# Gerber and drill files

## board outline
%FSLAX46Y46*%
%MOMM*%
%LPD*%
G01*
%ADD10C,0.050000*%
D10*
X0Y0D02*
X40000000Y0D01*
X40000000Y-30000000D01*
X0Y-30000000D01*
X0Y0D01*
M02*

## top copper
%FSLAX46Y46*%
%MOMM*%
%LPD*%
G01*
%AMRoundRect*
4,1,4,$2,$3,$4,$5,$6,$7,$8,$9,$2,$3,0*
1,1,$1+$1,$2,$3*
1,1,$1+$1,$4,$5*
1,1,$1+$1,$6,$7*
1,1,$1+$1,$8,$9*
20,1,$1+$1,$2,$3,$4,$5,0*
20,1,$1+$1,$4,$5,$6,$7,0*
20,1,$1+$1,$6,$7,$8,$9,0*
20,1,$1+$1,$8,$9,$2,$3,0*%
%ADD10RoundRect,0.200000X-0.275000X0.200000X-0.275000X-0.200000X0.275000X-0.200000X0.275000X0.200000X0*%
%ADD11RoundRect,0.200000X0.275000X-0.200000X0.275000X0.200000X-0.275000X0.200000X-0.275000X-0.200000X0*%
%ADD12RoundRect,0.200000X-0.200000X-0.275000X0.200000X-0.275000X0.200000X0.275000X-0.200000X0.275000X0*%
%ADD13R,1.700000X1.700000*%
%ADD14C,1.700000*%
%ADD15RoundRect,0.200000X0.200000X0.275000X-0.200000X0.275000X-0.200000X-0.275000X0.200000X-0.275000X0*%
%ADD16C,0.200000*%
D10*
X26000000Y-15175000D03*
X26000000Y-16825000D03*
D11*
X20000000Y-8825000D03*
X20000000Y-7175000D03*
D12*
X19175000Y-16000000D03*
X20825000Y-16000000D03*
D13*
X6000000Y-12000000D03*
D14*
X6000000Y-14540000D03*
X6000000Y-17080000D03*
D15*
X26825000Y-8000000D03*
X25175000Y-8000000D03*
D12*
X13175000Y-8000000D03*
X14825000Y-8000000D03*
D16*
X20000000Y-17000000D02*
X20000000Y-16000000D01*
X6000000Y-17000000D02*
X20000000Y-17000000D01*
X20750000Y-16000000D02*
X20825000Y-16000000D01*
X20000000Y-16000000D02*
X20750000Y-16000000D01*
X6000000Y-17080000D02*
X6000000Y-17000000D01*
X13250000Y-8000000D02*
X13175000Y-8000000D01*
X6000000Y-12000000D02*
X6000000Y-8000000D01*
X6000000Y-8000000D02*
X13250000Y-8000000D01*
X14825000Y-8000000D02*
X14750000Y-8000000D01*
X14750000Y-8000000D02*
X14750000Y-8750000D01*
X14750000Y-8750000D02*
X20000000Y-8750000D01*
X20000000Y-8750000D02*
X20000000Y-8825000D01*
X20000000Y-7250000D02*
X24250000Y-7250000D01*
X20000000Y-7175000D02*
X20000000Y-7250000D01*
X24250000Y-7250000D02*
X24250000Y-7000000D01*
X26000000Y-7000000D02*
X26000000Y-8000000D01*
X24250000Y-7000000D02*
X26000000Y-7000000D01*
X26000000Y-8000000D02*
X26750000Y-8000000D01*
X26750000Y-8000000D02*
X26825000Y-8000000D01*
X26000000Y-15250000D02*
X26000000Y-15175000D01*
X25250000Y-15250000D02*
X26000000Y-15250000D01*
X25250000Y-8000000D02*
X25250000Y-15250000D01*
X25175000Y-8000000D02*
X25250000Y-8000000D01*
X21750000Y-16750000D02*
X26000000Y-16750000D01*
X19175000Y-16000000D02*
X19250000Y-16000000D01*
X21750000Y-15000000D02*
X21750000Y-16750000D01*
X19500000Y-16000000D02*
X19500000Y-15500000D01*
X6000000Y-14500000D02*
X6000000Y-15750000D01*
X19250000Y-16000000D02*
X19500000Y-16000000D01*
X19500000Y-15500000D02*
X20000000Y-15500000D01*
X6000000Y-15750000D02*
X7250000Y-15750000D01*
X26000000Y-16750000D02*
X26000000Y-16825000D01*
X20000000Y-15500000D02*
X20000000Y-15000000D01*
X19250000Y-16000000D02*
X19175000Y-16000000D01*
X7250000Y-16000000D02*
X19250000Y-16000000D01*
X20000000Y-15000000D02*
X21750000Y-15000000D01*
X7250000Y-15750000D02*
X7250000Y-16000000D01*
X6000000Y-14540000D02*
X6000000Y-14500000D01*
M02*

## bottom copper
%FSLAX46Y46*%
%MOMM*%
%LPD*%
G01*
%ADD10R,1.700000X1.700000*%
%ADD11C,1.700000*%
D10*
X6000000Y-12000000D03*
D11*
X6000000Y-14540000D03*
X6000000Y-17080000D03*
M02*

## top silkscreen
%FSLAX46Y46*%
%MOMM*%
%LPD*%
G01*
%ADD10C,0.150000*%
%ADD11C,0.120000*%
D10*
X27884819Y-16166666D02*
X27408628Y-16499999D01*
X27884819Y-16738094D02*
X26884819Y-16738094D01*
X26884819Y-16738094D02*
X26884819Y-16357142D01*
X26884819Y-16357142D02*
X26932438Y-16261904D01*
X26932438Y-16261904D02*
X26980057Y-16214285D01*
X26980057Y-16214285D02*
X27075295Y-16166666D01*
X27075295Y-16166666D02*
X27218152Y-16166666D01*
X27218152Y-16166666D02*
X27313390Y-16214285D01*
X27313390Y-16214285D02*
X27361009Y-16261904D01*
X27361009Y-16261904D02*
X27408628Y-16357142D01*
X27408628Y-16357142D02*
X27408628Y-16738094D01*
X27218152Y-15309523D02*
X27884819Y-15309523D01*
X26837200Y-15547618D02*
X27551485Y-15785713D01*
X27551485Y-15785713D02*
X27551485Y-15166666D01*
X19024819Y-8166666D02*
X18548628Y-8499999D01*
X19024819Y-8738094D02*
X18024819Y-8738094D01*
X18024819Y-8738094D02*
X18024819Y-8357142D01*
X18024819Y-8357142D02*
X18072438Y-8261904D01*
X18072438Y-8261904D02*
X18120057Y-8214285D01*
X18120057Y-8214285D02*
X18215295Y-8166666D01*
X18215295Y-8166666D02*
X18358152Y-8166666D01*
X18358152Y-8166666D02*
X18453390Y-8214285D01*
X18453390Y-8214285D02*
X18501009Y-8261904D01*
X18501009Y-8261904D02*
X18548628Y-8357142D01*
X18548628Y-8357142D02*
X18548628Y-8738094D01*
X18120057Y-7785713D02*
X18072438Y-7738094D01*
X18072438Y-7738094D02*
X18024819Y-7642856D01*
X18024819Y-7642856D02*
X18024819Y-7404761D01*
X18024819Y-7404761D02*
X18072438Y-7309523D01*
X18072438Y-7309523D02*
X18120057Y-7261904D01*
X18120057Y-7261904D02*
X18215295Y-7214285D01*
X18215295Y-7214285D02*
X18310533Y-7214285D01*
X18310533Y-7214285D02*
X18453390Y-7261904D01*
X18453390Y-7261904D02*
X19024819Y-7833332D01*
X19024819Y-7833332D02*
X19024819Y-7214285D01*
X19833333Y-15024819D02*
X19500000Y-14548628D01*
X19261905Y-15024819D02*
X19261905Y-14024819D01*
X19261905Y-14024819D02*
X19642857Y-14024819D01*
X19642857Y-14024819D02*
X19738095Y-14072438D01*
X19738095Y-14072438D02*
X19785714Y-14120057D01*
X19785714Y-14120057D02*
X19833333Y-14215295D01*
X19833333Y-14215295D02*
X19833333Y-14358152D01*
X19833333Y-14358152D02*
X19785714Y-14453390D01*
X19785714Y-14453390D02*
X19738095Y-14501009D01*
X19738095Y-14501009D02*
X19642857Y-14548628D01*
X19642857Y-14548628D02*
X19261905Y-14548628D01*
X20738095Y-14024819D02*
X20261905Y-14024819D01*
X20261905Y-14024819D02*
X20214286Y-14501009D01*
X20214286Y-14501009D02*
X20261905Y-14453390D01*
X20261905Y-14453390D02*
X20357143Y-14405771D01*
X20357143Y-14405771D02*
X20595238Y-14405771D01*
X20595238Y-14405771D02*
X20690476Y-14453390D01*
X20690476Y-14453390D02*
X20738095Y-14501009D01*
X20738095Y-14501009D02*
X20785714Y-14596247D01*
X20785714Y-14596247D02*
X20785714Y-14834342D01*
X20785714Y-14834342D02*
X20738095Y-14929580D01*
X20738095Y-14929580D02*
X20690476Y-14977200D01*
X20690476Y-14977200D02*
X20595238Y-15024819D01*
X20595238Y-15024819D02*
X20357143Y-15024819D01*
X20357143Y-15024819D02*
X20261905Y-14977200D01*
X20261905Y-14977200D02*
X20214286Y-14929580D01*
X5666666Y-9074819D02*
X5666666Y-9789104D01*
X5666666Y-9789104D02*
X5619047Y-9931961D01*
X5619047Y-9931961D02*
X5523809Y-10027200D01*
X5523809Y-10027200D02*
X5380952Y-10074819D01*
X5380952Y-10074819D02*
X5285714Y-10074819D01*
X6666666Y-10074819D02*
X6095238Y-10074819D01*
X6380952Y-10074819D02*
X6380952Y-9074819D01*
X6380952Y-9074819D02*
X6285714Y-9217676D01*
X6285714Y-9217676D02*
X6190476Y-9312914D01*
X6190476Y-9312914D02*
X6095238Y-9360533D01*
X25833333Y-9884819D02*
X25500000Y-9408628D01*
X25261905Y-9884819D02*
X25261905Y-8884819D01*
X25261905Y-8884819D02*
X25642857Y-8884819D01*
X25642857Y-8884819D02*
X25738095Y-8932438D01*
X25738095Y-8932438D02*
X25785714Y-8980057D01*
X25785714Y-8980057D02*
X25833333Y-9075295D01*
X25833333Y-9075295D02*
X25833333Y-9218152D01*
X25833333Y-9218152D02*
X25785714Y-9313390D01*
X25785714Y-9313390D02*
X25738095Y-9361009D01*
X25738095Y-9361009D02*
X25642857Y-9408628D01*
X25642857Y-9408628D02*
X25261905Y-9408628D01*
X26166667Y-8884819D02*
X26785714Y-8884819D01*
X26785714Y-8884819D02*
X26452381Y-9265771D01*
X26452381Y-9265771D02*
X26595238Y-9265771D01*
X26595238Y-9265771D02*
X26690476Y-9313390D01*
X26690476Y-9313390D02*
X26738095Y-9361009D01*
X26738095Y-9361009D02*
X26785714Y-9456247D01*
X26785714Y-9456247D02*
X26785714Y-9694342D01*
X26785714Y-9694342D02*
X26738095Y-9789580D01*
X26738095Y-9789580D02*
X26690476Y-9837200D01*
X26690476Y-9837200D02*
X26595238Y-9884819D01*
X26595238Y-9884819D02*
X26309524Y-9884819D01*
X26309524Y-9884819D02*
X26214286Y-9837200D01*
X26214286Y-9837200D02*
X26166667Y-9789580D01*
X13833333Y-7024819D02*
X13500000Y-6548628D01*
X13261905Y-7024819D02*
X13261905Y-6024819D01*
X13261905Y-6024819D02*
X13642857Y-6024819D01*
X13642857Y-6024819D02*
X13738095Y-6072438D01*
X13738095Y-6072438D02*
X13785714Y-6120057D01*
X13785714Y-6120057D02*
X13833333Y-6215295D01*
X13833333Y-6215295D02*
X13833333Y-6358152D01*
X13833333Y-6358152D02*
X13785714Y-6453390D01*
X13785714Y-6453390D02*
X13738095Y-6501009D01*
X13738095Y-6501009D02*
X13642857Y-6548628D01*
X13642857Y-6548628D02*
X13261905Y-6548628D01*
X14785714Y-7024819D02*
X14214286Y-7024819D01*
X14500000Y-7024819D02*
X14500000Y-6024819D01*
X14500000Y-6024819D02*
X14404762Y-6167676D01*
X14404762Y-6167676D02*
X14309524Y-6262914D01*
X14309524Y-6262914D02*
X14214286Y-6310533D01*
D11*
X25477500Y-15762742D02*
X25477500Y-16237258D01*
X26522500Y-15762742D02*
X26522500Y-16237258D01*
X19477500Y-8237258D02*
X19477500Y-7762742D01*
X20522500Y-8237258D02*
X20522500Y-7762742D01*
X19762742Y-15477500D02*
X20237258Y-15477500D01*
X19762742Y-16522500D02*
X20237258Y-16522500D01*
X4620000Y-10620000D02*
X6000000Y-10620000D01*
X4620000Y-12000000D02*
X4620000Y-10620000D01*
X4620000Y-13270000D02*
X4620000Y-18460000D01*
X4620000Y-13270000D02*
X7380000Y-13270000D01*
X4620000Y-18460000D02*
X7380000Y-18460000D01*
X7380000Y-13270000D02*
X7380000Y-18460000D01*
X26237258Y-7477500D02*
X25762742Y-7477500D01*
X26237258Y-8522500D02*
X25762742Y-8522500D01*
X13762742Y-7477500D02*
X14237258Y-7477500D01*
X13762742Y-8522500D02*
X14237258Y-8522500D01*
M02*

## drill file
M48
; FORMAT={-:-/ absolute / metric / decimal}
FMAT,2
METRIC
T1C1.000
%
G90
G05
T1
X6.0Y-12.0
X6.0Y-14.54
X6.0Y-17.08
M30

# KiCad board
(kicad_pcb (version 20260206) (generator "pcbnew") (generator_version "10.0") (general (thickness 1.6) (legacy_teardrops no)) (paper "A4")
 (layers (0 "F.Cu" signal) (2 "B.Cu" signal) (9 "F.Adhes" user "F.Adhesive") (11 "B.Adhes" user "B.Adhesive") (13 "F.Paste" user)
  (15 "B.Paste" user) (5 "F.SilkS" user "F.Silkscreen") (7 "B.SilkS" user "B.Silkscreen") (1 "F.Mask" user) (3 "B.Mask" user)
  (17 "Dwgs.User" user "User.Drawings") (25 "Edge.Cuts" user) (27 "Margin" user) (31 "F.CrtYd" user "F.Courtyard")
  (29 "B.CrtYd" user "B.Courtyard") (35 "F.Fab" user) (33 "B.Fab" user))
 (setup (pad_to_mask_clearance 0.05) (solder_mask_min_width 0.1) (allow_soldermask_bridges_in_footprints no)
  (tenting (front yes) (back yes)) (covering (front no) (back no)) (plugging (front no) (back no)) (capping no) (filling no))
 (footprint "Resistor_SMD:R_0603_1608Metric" (layer "F.Cu") (at 26 16 -90)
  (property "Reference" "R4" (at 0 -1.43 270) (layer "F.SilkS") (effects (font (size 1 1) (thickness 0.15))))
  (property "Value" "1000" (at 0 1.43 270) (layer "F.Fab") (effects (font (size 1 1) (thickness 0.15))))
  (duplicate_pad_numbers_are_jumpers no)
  (fp_line (start -0.237258 0.5225) (end 0.237258 0.5225) (stroke (width 0.12) (type solid)) (layer "F.SilkS"))
  (fp_line (start -0.237258 -0.5225) (end 0.237258 -0.5225) (stroke (width 0.12) (type solid)) (layer "F.SilkS"))
  (pad "1" smd roundrect (at -0.825 0 270) (size 0.8 0.95) (layers "F.Cu" "F.Mask" "F.Paste") (roundrect_rratio 0.25) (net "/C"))
  (pad "2" smd roundrect (at 0.825 0 270) (size 0.8 0.95) (layers "F.Cu" "F.Mask" "F.Paste") (roundrect_rratio 0.25) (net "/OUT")))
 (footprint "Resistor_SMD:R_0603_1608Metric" (layer "F.Cu") (at 20 8 90)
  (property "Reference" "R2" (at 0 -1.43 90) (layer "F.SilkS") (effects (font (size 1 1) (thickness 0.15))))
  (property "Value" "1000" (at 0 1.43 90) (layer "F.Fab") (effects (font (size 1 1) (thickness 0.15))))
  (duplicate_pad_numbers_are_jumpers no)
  (fp_line (start -0.237258 -0.5225) (end 0.237258 -0.5225) (stroke (width 0.12) (type solid)) (layer "F.SilkS"))
  (fp_line (start -0.237258 0.5225) (end 0.237258 0.5225) (stroke (width 0.12) (type solid)) (layer "F.SilkS"))
  (pad "1" smd roundrect (at -0.825 0 90) (size 0.8 0.95) (layers "F.Cu" "F.Mask" "F.Paste") (roundrect_rratio 0.25) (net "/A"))
  (pad "2" smd roundrect (at 0.825 0 90) (size 0.8 0.95) (layers "F.Cu" "F.Mask" "F.Paste") (roundrect_rratio 0.25) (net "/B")))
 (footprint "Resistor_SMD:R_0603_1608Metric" (layer "F.Cu") (at 20 16)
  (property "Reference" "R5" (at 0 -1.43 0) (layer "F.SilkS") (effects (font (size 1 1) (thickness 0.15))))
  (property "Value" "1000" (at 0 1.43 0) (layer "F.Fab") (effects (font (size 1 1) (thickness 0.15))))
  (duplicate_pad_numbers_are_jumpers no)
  (fp_line (start -0.237258 -0.5225) (end 0.237258 -0.5225) (stroke (width 0.12) (type solid)) (layer "F.SilkS"))
  (fp_line (start -0.237258 0.5225) (end 0.237258 0.5225) (stroke (width 0.12) (type solid)) (layer "F.SilkS"))
  (pad "1" smd roundrect (at -0.825 0) (size 0.8 0.95) (layers "F.Cu" "F.Mask" "F.Paste") (roundrect_rratio 0.25) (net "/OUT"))
  (pad "2" smd roundrect (at 0.825 0) (size 0.8 0.95) (layers "F.Cu" "F.Mask" "F.Paste") (roundrect_rratio 0.25) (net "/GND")))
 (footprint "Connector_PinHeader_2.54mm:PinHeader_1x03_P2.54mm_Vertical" (layer "F.Cu") (at 6 12)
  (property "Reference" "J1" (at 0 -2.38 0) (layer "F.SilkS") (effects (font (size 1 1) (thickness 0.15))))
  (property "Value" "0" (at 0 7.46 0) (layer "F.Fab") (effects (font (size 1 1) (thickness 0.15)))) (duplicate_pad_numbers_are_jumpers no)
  (fp_line (start -1.38 -1.38) (end 0 -1.38) (stroke (width 0.12) (type solid)) (layer "F.SilkS"))
  (fp_line (start -1.38 0) (end -1.38 -1.38) (stroke (width 0.12) (type solid)) (layer "F.SilkS"))
  (fp_line (start -1.38 1.27) (end -1.38 6.46) (stroke (width 0.12) (type solid)) (layer "F.SilkS"))
  (fp_line (start -1.38 1.27) (end 1.38 1.27) (stroke (width 0.12) (type solid)) (layer "F.SilkS"))
  (fp_line (start -1.38 6.46) (end 1.38 6.46) (stroke (width 0.12) (type solid)) (layer "F.SilkS"))
  (fp_line (start 1.38 1.27) (end 1.38 6.46) (stroke (width 0.12) (type solid)) (layer "F.SilkS"))
  (pad "1" thru_hole rect (at 0 0) (size 1.7 1.7) (drill 1) (layers "*.Cu" "*.Mask") (remove_unused_layers no) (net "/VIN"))
  (pad "2" thru_hole circle (at 0 2.54) (size 1.7 1.7) (drill 1) (layers "*.Cu" "*.Mask") (remove_unused_layers no) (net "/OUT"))
  (pad "3" thru_hole circle (at 0 5.08) (size 1.7 1.7) (drill 1) (layers "*.Cu" "*.Mask") (remove_unused_layers no) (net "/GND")))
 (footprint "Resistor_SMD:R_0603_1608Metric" (layer "F.Cu") (at 26 8 180)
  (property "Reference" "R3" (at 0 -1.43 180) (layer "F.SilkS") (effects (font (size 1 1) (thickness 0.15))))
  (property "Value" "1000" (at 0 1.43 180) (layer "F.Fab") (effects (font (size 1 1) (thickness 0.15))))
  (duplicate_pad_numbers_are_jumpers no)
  (fp_line (start -0.237258 0.5225) (end 0.237258 0.5225) (stroke (width 0.12) (type solid)) (layer "F.SilkS"))
  (fp_line (start -0.237258 -0.5225) (end 0.237258 -0.5225) (stroke (width 0.12) (type solid)) (layer "F.SilkS"))
  (pad "1" smd roundrect (at -0.825 0 180) (size 0.8 0.95) (layers "F.Cu" "F.Mask" "F.Paste") (roundrect_rratio 0.25) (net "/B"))
  (pad "2" smd roundrect (at 0.825 0 180) (size 0.8 0.95) (layers "F.Cu" "F.Mask" "F.Paste") (roundrect_rratio 0.25) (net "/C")))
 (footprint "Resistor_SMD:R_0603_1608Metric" (layer "F.Cu") (at 14 8)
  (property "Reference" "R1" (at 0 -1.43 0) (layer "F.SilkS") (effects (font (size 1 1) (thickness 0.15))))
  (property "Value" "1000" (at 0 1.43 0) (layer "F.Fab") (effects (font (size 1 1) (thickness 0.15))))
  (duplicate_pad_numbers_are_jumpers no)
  (fp_line (start -0.237258 -0.5225) (end 0.237258 -0.5225) (stroke (width 0.12) (type solid)) (layer "F.SilkS"))
  (fp_line (start -0.237258 0.5225) (end 0.237258 0.5225) (stroke (width 0.12) (type solid)) (layer "F.SilkS"))
  (pad "1" smd roundrect (at -0.825 0) (size 0.8 0.95) (layers "F.Cu" "F.Mask" "F.Paste") (roundrect_rratio 0.25) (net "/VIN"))
  (pad "2" smd roundrect (at 0.825 0) (size 0.8 0.95) (layers "F.Cu" "F.Mask" "F.Paste") (roundrect_rratio 0.25) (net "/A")))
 (gr_rect (start 0 0) (end 40 30) (stroke (width 0.05) (type default)) (fill no) (layer "Edge.Cuts"))
 (segment (start 20 17) (end 20 16) (width 0.2) (layer "F.Cu") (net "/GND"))
 (segment (start 6 17) (end 20 17) (width 0.2) (layer "F.Cu") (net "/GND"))
 (segment (start 20.75 16) (end 20.825 16) (width 0.2) (layer "F.Cu") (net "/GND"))
 (segment (start 20 16) (end 20.75 16) (width 0.2) (layer "F.Cu") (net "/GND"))
 (segment (start 6 17.08) (end 6 17) (width 0.2) (layer "F.Cu") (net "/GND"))
 (segment (start 13.25 8) (end 13.175 8) (width 0.2) (layer "F.Cu") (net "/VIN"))
 (segment (start 6 12) (end 6 8) (width 0.2) (layer "F.Cu") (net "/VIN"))
 (segment (start 6 8) (end 13.25 8) (width 0.2) (layer "F.Cu") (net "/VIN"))
 (segment (start 14.825 8) (end 14.75 8) (width 0.2) (layer "F.Cu") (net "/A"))
 (segment (start 14.75 8) (end 14.75 8.75) (width 0.2) (layer "F.Cu") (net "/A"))
 (segment (start 14.75 8.75) (end 20 8.75) (width 0.2) (layer "F.Cu") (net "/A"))
 (segment (start 20 8.75) (end 20 8.825) (width 0.2) (layer "F.Cu") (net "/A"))
 (segment (start 20 7.25) (end 24.25 7.25) (width 0.2) (layer "F.Cu") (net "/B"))
 (segment (start 20 7.175) (end 20 7.25) (width 0.2) (layer "F.Cu") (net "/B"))
 (segment (start 24.25 7.25) (end 24.25 7) (width 0.2) (layer "F.Cu") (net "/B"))
 (segment (start 26 7) (end 26 8) (width 0.2) (layer "F.Cu") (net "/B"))
 (segment (start 24.25 7) (end 26 7) (width 0.2) (layer "F.Cu") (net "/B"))
 (segment (start 26 8) (end 26.75 8) (width 0.2) (layer "F.Cu") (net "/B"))
 (segment (start 26.75 8) (end 26.825 8) (width 0.2) (layer "F.Cu") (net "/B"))
 (segment (start 26 15.25) (end 26 15.175) (width 0.2) (layer "F.Cu") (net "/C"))
 (segment (start 25.25 15.25) (end 26 15.25) (width 0.2) (layer "F.Cu") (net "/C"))
 (segment (start 25.25 8) (end 25.25 15.25) (width 0.2) (layer "F.Cu") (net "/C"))
 (segment (start 25.175 8) (end 25.25 8) (width 0.2) (layer "F.Cu") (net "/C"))
 (segment (start 21.75 16.75) (end 26 16.75) (width 0.2) (layer "F.Cu") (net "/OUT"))
 (segment (start 19.175 16) (end 19.25 16) (width 0.2) (layer "F.Cu") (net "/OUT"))
 (segment (start 21.75 15) (end 21.75 16.75) (width 0.2) (layer "F.Cu") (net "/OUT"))
 (segment (start 19.5 16) (end 19.5 15.5) (width 0.2) (layer "F.Cu") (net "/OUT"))
 (segment (start 6 14.5) (end 6 15.75) (width 0.2) (layer "F.Cu") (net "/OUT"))
 (segment (start 19.25 16) (end 19.5 16) (width 0.2) (layer "F.Cu") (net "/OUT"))
 (segment (start 19.5 15.5) (end 20 15.5) (width 0.2) (layer "F.Cu") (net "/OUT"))
 (segment (start 6 15.75) (end 7.25 15.75) (width 0.2) (layer "F.Cu") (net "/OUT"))
 (segment (start 26 16.75) (end 26 16.825) (width 0.2) (layer "F.Cu") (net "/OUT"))
 (segment (start 20 15.5) (end 20 15) (width 0.2) (layer "F.Cu") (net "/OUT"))
 (segment (start 19.25 16) (end 19.175 16) (width 0.2) (layer "F.Cu") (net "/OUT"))
 (segment (start 7.25 16) (end 19.25 16) (width 0.2) (layer "F.Cu") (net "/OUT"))
 (segment (start 20 15) (end 21.75 15) (width 0.2) (layer "F.Cu") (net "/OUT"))
 (segment (start 7.25 15.75) (end 7.25 16) (width 0.2) (layer "F.Cu") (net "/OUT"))
 (segment (start 6 14.54) (end 6 14.5) (width 0.2) (layer "F.Cu") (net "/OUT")))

